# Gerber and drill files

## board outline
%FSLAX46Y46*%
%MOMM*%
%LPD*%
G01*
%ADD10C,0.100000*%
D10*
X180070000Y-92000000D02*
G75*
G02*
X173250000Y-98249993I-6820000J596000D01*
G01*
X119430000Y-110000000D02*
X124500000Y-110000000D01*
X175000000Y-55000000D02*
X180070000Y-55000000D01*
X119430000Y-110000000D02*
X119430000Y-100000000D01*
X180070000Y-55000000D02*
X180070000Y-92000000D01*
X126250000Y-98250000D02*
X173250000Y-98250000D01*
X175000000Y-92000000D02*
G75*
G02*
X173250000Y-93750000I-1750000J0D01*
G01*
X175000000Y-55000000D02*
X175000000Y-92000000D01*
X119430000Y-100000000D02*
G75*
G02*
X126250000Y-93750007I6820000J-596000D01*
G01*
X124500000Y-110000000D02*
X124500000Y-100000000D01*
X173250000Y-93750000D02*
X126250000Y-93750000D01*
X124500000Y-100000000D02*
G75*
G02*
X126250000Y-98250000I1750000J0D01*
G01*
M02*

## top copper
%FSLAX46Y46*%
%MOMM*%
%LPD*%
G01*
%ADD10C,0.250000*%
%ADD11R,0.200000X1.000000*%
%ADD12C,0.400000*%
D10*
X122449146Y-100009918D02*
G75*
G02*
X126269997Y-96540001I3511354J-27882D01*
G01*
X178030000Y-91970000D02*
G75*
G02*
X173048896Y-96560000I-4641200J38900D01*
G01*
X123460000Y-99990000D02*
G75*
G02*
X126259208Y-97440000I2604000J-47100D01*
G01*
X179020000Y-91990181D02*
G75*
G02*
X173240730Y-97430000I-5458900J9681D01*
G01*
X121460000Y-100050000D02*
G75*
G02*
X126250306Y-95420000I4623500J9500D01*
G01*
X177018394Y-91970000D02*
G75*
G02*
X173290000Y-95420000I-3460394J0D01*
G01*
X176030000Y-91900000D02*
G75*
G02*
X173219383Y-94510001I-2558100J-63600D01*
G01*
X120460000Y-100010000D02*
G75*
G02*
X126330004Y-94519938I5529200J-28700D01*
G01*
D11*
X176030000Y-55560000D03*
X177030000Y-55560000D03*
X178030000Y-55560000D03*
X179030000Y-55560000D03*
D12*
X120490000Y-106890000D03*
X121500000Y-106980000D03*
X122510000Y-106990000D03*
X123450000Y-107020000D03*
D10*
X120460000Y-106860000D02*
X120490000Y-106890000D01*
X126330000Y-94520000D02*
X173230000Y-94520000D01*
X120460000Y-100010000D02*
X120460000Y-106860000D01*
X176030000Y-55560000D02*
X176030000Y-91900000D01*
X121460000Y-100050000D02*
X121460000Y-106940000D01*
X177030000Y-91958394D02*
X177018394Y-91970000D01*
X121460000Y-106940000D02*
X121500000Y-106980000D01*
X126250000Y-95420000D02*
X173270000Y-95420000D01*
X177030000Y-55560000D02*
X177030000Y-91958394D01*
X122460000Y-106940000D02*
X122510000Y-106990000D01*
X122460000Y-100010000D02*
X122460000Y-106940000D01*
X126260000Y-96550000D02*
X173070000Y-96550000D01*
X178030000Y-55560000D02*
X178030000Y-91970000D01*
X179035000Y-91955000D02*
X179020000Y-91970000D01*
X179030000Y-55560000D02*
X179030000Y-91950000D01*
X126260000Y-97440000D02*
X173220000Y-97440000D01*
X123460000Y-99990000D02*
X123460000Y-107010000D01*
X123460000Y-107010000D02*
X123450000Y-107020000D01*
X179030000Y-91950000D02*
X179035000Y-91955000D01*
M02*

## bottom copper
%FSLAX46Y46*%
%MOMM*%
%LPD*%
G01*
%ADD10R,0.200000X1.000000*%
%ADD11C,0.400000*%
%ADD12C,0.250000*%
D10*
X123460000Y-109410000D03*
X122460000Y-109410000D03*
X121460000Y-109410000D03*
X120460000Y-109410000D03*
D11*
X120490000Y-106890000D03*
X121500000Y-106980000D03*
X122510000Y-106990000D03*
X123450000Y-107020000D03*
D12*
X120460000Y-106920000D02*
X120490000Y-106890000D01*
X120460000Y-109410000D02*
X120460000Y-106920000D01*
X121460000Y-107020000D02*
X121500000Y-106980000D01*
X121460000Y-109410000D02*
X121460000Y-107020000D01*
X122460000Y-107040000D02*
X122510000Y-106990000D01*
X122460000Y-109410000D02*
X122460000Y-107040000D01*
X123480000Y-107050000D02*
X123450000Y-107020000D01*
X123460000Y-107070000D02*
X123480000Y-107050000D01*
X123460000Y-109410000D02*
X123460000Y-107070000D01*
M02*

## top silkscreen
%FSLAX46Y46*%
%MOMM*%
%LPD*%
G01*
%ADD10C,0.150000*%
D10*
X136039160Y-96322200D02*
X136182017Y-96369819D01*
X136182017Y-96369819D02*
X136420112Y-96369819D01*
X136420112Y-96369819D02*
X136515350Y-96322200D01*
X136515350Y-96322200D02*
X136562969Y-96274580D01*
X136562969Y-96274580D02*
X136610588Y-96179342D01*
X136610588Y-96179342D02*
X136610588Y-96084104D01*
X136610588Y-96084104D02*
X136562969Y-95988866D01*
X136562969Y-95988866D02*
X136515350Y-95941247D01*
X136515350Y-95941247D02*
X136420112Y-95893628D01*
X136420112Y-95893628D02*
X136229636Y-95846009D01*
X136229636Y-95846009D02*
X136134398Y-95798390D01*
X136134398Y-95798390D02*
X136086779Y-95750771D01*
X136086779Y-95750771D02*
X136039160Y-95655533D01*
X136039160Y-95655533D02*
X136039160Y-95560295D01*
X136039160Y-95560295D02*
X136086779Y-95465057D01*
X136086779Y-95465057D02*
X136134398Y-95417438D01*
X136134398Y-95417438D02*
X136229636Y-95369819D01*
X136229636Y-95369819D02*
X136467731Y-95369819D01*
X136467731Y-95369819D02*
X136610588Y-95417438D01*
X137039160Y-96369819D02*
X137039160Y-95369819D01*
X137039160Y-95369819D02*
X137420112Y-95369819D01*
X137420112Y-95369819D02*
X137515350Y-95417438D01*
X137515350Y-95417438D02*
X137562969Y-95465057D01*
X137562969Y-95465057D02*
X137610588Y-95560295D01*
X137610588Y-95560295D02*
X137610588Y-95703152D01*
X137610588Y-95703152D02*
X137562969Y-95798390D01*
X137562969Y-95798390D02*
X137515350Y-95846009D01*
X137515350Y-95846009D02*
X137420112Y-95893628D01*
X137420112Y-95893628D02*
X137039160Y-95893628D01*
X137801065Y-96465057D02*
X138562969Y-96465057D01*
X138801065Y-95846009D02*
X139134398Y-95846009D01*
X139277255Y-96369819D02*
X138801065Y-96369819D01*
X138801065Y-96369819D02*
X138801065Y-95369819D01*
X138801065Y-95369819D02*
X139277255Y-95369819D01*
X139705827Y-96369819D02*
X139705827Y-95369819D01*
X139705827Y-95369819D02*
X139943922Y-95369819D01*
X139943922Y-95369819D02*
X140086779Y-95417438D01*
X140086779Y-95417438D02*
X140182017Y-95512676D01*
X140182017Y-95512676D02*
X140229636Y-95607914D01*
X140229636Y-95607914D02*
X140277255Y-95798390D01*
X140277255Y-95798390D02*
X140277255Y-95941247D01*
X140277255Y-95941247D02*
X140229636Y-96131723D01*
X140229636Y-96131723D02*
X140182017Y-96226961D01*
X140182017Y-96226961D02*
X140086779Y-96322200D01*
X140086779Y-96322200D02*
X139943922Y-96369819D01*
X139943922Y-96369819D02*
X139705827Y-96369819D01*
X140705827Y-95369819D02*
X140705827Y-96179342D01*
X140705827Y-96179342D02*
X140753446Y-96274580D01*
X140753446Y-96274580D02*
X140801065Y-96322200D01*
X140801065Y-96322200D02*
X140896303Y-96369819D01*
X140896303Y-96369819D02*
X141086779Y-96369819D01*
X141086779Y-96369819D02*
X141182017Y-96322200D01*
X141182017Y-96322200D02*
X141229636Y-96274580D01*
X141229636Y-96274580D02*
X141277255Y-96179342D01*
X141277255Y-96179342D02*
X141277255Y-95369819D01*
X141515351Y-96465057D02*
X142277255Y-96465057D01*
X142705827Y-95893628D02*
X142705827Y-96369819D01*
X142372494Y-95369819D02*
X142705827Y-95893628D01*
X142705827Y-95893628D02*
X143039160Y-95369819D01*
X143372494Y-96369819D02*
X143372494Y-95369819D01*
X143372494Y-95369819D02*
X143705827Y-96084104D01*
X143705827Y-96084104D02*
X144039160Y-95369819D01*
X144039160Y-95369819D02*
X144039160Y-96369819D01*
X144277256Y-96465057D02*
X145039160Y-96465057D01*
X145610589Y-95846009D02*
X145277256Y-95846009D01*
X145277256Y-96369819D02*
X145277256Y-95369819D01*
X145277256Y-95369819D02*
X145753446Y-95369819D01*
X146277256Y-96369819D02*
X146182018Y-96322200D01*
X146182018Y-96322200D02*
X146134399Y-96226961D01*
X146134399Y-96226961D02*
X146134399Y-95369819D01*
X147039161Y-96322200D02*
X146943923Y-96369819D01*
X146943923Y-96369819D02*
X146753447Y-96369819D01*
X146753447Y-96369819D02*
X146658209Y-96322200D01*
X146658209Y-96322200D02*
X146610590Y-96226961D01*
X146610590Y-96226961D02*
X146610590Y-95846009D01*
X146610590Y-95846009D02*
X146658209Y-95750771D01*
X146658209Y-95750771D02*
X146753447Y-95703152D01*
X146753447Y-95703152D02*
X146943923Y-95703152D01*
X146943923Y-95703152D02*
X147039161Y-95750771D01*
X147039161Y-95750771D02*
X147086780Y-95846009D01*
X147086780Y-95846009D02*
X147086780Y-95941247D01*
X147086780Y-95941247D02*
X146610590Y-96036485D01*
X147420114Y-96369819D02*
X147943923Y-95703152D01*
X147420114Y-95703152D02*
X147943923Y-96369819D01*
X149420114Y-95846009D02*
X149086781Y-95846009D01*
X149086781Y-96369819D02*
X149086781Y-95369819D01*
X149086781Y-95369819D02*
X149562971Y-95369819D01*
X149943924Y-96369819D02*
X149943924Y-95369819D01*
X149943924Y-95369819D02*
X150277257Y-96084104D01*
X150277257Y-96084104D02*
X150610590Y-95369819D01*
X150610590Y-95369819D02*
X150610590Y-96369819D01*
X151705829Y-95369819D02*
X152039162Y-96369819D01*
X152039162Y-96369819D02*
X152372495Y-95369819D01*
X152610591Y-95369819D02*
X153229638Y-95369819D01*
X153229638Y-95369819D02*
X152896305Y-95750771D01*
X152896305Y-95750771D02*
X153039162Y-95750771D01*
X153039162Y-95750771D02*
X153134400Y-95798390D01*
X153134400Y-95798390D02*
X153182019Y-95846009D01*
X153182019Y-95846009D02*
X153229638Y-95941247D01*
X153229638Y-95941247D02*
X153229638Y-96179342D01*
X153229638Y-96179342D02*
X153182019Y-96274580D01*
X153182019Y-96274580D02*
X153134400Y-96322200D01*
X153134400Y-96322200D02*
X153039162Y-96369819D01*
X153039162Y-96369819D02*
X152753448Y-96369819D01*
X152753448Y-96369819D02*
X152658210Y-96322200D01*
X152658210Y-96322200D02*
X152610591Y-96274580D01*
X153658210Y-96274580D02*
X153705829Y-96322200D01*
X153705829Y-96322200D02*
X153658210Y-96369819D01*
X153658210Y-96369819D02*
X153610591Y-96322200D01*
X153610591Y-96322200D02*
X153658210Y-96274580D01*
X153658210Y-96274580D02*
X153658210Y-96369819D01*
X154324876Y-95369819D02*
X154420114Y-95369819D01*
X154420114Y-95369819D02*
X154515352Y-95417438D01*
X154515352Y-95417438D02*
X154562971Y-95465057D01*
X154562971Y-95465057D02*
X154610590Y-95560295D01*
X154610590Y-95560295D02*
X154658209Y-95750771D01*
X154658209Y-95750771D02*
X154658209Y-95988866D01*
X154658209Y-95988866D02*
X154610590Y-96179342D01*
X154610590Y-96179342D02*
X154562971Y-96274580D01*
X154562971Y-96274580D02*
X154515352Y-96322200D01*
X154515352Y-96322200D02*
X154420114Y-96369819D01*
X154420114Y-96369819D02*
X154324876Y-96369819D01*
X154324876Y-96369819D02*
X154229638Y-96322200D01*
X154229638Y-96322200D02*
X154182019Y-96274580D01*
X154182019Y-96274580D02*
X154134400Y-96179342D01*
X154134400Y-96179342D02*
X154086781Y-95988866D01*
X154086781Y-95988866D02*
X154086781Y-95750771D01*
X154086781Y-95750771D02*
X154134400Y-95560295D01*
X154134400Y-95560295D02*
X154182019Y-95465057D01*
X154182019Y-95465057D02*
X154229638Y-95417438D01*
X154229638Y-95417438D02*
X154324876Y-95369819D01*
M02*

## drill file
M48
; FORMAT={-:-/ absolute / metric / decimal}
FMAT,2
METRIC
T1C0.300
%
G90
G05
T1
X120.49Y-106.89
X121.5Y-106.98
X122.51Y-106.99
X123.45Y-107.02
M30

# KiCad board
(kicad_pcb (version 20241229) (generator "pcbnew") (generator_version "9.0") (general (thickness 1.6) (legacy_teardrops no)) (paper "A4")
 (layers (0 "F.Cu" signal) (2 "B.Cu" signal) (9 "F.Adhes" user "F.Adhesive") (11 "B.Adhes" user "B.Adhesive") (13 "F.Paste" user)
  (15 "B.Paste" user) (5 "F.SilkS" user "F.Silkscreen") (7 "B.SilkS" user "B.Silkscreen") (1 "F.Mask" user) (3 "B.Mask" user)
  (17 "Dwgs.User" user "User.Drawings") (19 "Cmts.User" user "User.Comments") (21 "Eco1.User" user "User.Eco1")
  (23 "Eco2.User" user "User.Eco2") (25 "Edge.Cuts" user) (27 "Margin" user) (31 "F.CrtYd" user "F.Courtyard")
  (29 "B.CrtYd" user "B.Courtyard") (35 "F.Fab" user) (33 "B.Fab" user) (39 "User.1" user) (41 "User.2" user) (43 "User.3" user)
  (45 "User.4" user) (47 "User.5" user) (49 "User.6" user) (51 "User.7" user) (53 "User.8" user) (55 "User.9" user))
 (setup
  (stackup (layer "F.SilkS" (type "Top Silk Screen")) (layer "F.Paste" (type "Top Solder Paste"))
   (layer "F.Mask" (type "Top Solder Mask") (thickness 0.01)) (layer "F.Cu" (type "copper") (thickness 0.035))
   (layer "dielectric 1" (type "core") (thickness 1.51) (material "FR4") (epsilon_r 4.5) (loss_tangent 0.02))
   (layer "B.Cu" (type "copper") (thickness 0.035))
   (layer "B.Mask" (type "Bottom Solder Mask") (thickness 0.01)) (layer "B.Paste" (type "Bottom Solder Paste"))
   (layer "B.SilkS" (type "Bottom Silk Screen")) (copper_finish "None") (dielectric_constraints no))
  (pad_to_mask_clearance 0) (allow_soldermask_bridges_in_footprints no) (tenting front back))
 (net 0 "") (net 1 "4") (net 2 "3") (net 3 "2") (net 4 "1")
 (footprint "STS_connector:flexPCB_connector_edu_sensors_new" (layer "F.Cu") (at 175.53 55.06)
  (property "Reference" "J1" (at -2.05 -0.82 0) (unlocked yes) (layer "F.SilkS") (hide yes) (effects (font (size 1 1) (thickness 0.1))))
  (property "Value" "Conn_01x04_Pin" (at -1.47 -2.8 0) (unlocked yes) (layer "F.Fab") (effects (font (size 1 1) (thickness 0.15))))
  (pad "1" smd rect (at 0.5 0.5) (size 0.2 1) (layers "F.Cu" "F.Mask" "F.Paste") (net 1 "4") (thermal_bridge_angle 45))
  (pad "2" smd rect (at 1.5 0.5) (size 0.2 1) (layers "F.Cu" "F.Mask" "F.Paste") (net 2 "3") (thermal_bridge_angle 45))
  (pad "3" smd rect (at 2.5 0.5) (size 0.2 1) (layers "F.Cu" "F.Mask" "F.Paste") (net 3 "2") (thermal_bridge_angle 45))
  (pad "4" smd rect (at 3.5 0.5) (size 0.2 1) (layers "F.Cu" "F.Mask" "F.Paste") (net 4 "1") (thermal_bridge_angle 45)))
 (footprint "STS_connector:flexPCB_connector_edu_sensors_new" (layer "B.Cu") (at 123.96 108.91 180)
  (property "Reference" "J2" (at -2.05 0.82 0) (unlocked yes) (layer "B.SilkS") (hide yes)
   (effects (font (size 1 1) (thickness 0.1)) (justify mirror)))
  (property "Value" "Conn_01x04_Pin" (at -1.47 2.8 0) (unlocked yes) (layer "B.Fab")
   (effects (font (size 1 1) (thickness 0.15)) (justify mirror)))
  (pad "1" smd rect (at 0.5 -0.5 180) (size 0.2 1) (layers "B.Cu" "B.Mask" "B.Paste") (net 4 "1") (thermal_bridge_angle 45))
  (pad "2" smd rect (at 1.5 -0.5 180) (size 0.2 1) (layers "B.Cu" "B.Mask" "B.Paste") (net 3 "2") (thermal_bridge_angle 45))
  (pad "3" smd rect (at 2.5 -0.5 180) (size 0.2 1) (layers "B.Cu" "B.Mask" "B.Paste") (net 2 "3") (thermal_bridge_angle 45))
  (pad "4" smd rect (at 3.5 -0.5 180) (size 0.2 1) (layers "B.Cu" "B.Mask" "B.Paste") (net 1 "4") (thermal_bridge_angle 45)))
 (gr_arc (start 122.449146 100.009918) (mid 123.599769 97.438313) (end 126.269997 96.540001) (stroke (width 0.25) (type solid))
  (layer "F.Cu") (net 3))
 (gr_arc (start 178.03 91.97) (mid 176.534005 95.344301) (end 173.048896 96.56) (stroke (width 0.25) (type solid)) (layer "F.Cu") (net 3))
 (gr_arc (start 123.46 99.99) (mid 124.310092 98.111785) (end 126.259208 97.44) (stroke (width 0.25) (type solid)) (layer "F.Cu") (net 4))
 (gr_arc (start 179.02 91.990181) (mid 177.302628 95.955504) (end 173.24073 97.43) (stroke (width 0.25) (type solid)) (layer "F.Cu") (net 4))
 (gr_arc (start 121.46 100.05) (mid 122.870284 96.716032) (end 126.250306 95.42) (stroke (width 0.25) (type solid)) (layer "F.Cu") (net 2))
 (gr_arc (start 177.018394 91.97) (mid 175.908206 94.509854) (end 173.29 95.42) (stroke (width 0.25) (type solid)) (layer "F.Cu") (net 2))
 (gr_arc (start 176.03 91.9) (mid 175.213151 93.838691) (end 173.219383 94.51) (stroke (width 0.25) (type solid)) (layer "F.Cu") (net 1))
 (gr_arc (start 120.46 100.01) (mid 122.212295 96.000431) (end 126.33 94.52) (stroke (width 0.25) (type solid)) (layer "F.Cu") (net 1))
 (gr_arc (start 180.07 92) (mid 177.875335 96.451174) (end 173.25 98.25) (stroke (width 0.1) (type default)) (layer "Edge.Cuts"))
 (gr_line (start 119.43 110) (end 124.5 110) (stroke (width 0.1) (type solid)) (layer "Edge.Cuts"))
 (gr_line (start 175 55) (end 180.07 55) (stroke (width 0.1) (type default)) (layer "Edge.Cuts"))
 (gr_line (start 119.43 110) (end 119.43 100) (stroke (width 0.1) (type solid)) (layer "Edge.Cuts"))
 (gr_line (start 180.07 55) (end 180.07 92) (stroke (width 0.1) (type solid)) (layer "Edge.Cuts"))
 (gr_line (start 126.25 98.25) (end 173.25 98.25) (stroke (width 0.1) (type default)) (layer "Edge.Cuts"))
 (gr_arc (start 175 92) (mid 174.487437 93.237437) (end 173.25 93.75) (stroke (width 0.1) (type default)) (layer "Edge.Cuts"))
 (gr_line (start 175 55) (end 175 92) (stroke (width 0.1) (type solid)) (layer "Edge.Cuts"))
 (gr_arc (start 119.43 100) (mid 121.624665 95.548826) (end 126.25 93.75) (stroke (width 0.1) (type default)) (layer "Edge.Cuts"))
 (gr_line (start 124.5 110) (end 124.5 100) (stroke (width 0.1) (type default)) (layer "Edge.Cuts"))
 (gr_line (start 173.25 93.75) (end 126.25 93.75) (stroke (width 0.1) (type default)) (layer "Edge.Cuts"))
 (gr_arc (start 124.5 100) (mid 125.012563 98.762563) (end 126.25 98.25) (stroke (width 0.1) (type default)) (layer "Edge.Cuts"))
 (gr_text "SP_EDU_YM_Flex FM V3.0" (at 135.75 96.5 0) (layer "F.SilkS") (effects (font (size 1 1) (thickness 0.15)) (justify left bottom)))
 (segment (start 120.46 106.86) (end 120.49 106.89) (width 0.25) (layer "F.Cu") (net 1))
 (segment (start 126.33 94.52) (end 173.23 94.52) (width 0.25) (layer "F.Cu") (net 1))
 (segment (start 120.46 100.01) (end 120.46 106.86) (width 0.25) (layer "F.Cu") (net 1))
 (segment (start 176.03 55.56) (end 176.03 91.9) (width 0.25) (layer "F.Cu") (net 1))
 (via (at 120.49 106.89) (size 0.4) (drill 0.3) (layers "F.Cu" "B.Cu") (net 1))
 (segment (start 120.46 106.92) (end 120.49 106.89) (width 0.25) (layer "B.Cu") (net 1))
 (segment (start 120.46 109.41) (end 120.46 106.92) (width 0.25) (layer "B.Cu") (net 1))
 (segment (start 121.46 100.05) (end 121.46 106.94) (width 0.25) (layer "F.Cu") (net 2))
 (segment (start 177.03 91.958394) (end 177.018394 91.97) (width 0.25) (layer "F.Cu") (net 2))
 (segment (start 121.46 106.94) (end 121.5 106.98) (width 0.25) (layer "F.Cu") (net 2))
 (segment (start 126.25 95.42) (end 173.27 95.42) (width 0.25) (layer "F.Cu") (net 2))
 (segment (start 177.03 55.56) (end 177.03 91.958394) (width 0.25) (layer "F.Cu") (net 2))
 (via (at 121.5 106.98) (size 0.4) (drill 0.3) (layers "F.Cu" "B.Cu") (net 2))
 (segment (start 121.46 107.02) (end 121.5 106.98) (width 0.25) (layer "B.Cu") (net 2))
 (segment (start 121.46 109.41) (end 121.46 107.02) (width 0.25) (layer "B.Cu") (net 2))
 (segment (start 122.46 106.94) (end 122.51 106.99) (width 0.25) (layer "F.Cu") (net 3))
 (segment (start 122.46 100.01) (end 122.46 106.94) (width 0.25) (layer "F.Cu") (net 3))
 (segment (start 126.26 96.55) (end 173.07 96.55) (width 0.25) (layer "F.Cu") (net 3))
 (segment (start 178.03 55.56) (end 178.03 91.97) (width 0.25) (layer "F.Cu") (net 3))
 (via (at 122.51 106.99) (size 0.4) (drill 0.3) (layers "F.Cu" "B.Cu") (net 3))
 (segment (start 122.46 107.04) (end 122.51 106.99) (width 0.25) (layer "B.Cu") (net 3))
 (segment (start 122.46 109.41) (end 122.46 107.04) (width 0.25) (layer "B.Cu") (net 3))
 (segment (start 179.035 91.955) (end 179.02 91.97) (width 0.25) (layer "F.Cu") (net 4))
 (segment (start 179.03 55.56) (end 179.03 91.95) (width 0.25) (layer "F.Cu") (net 4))
 (segment (start 126.26 97.44) (end 173.22 97.44) (width 0.25) (layer "F.Cu") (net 4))
 (segment (start 123.46 99.99) (end 123.46 107.01) (width 0.25) (layer "F.Cu") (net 4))
 (segment (start 123.46 107.01) (end 123.45 107.02) (width 0.25) (layer "F.Cu") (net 4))
 (segment (start 179.03 91.95) (end 179.035 91.955) (width 0.25) (layer "F.Cu") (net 4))
 (via (at 123.45 107.02) (size 0.4) (drill 0.3) (layers "F.Cu" "B.Cu") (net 4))
 (segment (start 123.48 107.05) (end 123.45 107.02) (width 0.25) (layer "B.Cu") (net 4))
 (segment (start 123.46 107.07) (end 123.48 107.05) (width 0.25) (layer "B.Cu") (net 4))
 (segment (start 123.46 109.41) (end 123.46 107.07) (width 0.25) (layer "B.Cu") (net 4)))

